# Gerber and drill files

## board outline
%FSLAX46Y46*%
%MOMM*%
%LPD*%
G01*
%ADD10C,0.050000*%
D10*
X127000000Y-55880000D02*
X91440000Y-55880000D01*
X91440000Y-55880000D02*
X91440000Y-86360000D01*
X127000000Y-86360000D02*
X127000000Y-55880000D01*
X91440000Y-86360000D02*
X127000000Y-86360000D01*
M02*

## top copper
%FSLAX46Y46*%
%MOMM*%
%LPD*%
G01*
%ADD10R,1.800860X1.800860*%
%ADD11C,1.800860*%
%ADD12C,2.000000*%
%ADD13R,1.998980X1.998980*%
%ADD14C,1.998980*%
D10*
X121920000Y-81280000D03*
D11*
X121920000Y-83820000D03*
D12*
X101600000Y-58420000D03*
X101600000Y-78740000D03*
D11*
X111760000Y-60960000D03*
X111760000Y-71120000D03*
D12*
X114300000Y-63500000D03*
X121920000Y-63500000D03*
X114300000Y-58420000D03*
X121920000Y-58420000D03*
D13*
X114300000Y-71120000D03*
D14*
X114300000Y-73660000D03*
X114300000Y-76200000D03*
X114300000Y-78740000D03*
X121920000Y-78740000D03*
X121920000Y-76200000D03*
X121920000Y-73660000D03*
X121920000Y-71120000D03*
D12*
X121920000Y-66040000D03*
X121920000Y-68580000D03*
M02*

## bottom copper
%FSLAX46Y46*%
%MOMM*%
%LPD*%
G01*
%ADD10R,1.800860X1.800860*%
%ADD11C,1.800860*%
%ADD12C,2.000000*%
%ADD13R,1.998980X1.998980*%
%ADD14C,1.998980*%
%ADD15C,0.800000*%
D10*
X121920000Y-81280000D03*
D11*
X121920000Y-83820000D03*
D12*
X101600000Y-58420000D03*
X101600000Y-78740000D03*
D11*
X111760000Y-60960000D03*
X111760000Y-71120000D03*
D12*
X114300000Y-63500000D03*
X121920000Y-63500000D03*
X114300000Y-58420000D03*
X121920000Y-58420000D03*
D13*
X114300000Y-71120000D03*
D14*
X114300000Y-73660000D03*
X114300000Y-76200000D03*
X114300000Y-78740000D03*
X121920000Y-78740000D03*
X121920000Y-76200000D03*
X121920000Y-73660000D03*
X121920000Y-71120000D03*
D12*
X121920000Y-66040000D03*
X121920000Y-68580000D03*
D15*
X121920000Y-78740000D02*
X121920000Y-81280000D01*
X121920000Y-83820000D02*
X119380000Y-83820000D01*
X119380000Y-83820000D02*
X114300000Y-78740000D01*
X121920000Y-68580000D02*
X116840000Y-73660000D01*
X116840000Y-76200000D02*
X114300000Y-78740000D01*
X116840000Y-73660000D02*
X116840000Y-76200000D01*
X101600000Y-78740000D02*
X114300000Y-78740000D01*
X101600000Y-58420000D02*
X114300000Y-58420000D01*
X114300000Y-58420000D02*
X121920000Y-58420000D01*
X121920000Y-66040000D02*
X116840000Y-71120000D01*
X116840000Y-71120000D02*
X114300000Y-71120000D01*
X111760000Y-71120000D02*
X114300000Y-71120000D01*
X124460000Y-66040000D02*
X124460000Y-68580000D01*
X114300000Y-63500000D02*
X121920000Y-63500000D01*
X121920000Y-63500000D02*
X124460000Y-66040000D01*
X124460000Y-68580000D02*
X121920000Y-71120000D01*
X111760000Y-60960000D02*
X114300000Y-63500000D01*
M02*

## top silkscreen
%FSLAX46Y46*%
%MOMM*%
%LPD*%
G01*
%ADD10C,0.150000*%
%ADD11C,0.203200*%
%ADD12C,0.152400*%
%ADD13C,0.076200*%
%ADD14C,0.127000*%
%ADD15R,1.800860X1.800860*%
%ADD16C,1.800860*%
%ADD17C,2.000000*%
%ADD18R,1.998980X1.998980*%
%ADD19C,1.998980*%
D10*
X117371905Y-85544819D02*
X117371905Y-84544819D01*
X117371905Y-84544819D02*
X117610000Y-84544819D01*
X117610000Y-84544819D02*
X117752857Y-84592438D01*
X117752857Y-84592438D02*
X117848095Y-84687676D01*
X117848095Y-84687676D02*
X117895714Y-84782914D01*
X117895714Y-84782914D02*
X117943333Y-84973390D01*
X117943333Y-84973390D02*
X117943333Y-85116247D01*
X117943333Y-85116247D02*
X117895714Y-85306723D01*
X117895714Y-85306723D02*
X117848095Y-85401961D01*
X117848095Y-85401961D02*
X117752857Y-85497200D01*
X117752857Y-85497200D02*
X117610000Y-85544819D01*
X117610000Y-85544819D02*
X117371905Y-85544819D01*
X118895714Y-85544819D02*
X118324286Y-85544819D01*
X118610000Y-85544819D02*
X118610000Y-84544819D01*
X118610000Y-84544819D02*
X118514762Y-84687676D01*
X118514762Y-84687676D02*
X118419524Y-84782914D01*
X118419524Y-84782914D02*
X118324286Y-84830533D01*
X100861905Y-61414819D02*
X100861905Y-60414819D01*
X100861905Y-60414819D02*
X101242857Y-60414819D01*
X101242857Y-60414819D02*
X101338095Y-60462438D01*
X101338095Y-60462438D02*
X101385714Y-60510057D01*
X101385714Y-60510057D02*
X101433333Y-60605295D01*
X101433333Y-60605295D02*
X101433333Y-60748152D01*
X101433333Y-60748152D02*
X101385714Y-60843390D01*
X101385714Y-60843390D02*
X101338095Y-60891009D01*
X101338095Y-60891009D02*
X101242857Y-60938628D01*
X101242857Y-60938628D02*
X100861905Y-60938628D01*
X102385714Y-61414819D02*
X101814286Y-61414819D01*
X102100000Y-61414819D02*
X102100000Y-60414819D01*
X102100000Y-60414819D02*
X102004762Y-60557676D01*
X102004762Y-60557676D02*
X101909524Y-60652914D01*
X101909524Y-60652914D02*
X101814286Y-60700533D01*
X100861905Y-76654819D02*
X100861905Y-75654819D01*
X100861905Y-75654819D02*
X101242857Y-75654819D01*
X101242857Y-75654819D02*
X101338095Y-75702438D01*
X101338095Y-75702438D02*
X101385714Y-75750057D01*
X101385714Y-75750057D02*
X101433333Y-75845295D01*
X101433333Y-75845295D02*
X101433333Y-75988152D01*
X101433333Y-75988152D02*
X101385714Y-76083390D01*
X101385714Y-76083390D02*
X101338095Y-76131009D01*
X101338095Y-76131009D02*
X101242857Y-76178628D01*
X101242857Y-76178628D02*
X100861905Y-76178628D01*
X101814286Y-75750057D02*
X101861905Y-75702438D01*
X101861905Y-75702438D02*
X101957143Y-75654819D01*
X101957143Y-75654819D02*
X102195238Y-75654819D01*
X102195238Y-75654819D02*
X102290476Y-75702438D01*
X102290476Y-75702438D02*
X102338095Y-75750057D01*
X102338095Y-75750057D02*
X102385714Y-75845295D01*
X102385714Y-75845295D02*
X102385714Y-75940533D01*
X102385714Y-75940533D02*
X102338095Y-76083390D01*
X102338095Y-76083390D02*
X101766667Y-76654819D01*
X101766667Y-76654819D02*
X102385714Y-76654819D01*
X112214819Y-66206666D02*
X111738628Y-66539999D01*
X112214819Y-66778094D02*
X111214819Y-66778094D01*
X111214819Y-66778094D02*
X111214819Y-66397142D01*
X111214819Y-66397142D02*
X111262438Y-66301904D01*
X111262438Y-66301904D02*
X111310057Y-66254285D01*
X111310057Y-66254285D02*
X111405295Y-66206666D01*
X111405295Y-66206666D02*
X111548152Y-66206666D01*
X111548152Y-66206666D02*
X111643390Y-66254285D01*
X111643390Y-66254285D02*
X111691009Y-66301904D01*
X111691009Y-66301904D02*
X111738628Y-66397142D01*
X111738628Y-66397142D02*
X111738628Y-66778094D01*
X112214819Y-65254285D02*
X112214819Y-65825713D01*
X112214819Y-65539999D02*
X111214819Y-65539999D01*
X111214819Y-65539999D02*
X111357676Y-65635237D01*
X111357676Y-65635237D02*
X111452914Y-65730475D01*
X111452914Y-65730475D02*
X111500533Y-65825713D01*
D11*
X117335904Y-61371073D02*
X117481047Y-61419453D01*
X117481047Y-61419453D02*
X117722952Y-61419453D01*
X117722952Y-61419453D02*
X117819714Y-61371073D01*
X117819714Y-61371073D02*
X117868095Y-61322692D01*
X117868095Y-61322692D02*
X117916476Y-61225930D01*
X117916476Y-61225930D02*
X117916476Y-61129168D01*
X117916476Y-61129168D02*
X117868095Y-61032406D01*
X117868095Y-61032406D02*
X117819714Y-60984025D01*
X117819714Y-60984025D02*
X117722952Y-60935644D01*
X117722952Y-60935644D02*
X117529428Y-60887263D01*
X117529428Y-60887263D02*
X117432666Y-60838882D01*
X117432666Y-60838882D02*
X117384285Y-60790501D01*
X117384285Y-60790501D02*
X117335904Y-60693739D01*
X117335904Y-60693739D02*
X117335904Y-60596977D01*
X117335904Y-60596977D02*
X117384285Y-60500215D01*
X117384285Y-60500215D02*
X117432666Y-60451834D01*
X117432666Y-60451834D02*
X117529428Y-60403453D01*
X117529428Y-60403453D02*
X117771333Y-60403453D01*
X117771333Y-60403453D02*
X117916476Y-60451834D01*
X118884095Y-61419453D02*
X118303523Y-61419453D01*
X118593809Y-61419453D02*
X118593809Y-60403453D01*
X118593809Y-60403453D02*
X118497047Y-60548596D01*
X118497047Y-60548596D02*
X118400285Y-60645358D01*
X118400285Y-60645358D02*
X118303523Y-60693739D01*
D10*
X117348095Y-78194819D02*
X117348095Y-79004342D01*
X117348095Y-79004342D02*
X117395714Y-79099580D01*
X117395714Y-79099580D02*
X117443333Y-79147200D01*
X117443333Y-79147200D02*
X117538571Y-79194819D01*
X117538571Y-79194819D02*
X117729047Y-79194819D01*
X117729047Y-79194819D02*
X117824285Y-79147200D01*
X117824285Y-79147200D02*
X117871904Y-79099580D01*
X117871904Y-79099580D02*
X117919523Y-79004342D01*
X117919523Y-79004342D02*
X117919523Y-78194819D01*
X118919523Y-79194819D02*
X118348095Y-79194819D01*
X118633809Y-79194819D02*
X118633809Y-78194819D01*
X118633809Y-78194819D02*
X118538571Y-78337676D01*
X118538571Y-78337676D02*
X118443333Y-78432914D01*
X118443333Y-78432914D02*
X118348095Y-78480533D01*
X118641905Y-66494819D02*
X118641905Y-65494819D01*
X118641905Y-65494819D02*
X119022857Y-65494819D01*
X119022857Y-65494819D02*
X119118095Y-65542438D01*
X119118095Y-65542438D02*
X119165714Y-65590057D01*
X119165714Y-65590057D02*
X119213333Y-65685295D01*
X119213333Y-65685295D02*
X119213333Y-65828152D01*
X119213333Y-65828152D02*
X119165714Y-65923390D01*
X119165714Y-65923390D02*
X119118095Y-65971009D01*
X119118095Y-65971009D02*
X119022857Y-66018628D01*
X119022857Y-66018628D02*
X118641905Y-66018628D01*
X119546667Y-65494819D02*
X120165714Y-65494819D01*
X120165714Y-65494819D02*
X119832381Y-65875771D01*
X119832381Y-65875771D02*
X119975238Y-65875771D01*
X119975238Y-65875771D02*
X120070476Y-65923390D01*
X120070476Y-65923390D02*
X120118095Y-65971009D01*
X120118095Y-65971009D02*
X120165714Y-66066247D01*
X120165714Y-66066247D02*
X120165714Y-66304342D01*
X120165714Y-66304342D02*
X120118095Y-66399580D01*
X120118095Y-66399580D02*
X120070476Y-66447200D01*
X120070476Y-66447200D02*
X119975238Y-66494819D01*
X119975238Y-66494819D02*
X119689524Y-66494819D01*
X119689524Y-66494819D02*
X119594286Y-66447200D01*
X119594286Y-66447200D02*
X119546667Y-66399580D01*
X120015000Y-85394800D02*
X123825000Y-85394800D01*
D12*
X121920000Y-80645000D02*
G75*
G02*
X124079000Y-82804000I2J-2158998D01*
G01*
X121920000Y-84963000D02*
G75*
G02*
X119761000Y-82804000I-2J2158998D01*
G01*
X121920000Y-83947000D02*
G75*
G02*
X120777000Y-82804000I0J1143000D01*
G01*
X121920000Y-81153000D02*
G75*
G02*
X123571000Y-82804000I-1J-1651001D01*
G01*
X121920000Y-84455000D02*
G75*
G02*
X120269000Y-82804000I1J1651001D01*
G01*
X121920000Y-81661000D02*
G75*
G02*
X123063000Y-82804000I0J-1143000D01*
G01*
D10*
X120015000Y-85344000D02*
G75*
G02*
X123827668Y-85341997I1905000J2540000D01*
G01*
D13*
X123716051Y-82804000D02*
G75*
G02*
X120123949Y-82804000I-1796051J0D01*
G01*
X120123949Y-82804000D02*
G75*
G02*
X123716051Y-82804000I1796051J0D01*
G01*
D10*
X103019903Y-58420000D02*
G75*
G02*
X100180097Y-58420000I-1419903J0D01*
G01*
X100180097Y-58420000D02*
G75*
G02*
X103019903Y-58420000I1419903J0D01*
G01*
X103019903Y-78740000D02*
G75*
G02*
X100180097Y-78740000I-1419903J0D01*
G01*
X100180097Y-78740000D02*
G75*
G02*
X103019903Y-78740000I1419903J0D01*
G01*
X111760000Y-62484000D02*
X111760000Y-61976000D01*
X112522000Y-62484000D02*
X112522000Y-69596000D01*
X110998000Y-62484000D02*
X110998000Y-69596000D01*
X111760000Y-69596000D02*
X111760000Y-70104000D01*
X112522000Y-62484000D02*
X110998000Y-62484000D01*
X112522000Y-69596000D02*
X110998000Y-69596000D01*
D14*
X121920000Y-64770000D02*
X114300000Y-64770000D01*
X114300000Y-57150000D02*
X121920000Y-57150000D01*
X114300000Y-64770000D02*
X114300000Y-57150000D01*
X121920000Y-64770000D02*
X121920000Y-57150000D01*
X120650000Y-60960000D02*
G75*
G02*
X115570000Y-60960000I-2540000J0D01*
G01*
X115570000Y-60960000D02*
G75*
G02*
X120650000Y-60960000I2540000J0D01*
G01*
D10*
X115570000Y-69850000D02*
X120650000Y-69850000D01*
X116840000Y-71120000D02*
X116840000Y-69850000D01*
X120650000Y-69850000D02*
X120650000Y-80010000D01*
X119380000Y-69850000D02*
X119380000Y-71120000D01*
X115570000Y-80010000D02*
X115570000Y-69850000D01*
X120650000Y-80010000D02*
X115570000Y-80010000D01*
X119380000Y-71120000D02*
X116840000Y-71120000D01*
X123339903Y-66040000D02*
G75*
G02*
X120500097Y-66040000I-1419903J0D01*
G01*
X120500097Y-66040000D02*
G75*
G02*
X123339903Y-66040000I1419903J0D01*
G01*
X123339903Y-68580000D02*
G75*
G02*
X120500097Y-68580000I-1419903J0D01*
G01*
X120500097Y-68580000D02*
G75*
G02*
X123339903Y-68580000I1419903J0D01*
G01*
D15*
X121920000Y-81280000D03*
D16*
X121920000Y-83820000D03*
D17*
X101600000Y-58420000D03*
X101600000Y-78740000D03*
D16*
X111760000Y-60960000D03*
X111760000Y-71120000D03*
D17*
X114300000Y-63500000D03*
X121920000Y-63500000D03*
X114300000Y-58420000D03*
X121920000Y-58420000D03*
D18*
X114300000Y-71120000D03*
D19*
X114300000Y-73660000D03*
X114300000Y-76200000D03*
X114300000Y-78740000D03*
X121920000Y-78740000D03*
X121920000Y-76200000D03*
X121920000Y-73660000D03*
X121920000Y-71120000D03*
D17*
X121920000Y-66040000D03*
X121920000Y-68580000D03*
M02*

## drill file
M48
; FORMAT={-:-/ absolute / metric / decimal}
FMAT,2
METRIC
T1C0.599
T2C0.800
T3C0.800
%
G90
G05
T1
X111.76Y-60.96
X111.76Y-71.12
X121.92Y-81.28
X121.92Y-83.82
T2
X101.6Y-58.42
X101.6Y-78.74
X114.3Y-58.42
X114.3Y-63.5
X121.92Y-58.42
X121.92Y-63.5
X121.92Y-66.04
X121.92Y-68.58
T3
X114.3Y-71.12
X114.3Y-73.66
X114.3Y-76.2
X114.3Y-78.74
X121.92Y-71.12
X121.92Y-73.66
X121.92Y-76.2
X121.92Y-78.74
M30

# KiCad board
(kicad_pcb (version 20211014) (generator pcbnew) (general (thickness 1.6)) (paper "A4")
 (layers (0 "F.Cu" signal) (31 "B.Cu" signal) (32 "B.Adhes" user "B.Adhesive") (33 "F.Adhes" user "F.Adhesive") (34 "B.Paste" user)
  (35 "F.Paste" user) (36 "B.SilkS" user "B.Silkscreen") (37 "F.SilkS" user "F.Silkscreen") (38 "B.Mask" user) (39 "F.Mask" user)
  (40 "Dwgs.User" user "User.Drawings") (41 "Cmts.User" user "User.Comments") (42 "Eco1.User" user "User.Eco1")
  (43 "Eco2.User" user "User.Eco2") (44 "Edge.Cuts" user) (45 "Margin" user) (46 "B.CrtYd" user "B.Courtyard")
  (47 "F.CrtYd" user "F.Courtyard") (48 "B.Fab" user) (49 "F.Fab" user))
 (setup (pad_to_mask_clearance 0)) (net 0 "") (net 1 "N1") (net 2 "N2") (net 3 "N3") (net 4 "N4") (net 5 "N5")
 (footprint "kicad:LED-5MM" (layer "F.Cu") (at 121.92 82.55 -90)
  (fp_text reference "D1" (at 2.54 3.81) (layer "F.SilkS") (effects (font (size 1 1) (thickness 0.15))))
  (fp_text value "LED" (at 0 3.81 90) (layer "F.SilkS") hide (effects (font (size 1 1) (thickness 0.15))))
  (fp_line (start 2.8448 1.905) (end 2.8448 -1.905) (layer "F.SilkS") (width 0.15))
  (fp_arc (start -1.905 0) (mid -1.272644 -1.526644) (end 0.254 -2.159) (layer "F.SilkS") (width 0.1524))
  (fp_arc (start 2.413 0) (mid 1.780644 1.526644) (end 0.254 2.159) (layer "F.SilkS") (width 0.1524))
  (fp_arc (start 1.397 0) (mid 1.062223 0.808223) (end 0.254 1.143) (layer "F.SilkS") (width 0.1524))
  (fp_arc (start -1.397 0) (mid -0.913433 -1.167433) (end 0.254 -1.651) (layer "F.SilkS") (width 0.1524))
  (fp_arc (start 1.905 0) (mid 1.421433 1.167433) (end 0.254 1.651) (layer "F.SilkS") (width 0.1524))
  (fp_arc (start -0.889 0) (mid -0.554223 -0.808223) (end 0.254 -1.143) (layer "F.SilkS") (width 0.1524))
  (fp_arc (start 2.794 1.905) (mid -2.921 0.001668) (end 2.791997 -1.907668) (layer "F.SilkS") (width 0.15))
  (fp_circle (center 0.254 0) (end -1.016 1.27) (layer "F.SilkS") (width 0.0762) (fill none))
  (pad "1" thru_hole rect locked (at -1.27 0 270) (size 1.80086 1.80086) (drill 0.59944) (layers *.Cu "F.Paste" "F.SilkS" "F.Mask")
   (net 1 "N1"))
  (pad "2" thru_hole circle locked (at 1.27 0 270) (size 1.80086 1.80086) (drill 0.59944) (layers *.Cu "F.Paste" "F.SilkS" "F.Mask")
   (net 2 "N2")))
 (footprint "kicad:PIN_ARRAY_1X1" (layer "F.Cu") (at 101.6 58.42)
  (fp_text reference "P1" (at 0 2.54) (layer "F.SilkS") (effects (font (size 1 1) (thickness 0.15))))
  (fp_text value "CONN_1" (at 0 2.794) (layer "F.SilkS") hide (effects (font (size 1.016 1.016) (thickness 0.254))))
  (fp_circle (center 0 0) (end 1.27 0.635) (layer "F.SilkS") (width 0.15) (fill none))
  (pad "1" thru_hole circle locked (at 0 0) (size 2 2) (drill 0.8) (layers *.Cu *.Mask "F.SilkS") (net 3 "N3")))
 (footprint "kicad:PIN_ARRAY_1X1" (layer "F.Cu") (at 101.6 78.74)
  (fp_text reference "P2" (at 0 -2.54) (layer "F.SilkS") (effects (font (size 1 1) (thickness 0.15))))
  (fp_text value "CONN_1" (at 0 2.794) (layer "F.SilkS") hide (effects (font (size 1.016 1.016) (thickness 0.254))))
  (fp_circle (center 0 0) (end 1.27 0.635) (layer "F.SilkS") (width 0.15) (fill none))
  (pad "1" thru_hole circle locked (at 0 0) (size 2 2) (drill 0.8) (layers *.Cu *.Mask "F.SilkS") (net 2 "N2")))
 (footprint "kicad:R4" (layer "F.Cu") (at 111.76 66.04 -90) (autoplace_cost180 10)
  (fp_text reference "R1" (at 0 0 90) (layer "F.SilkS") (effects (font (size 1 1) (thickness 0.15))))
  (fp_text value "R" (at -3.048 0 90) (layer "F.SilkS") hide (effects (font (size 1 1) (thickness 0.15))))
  (fp_line (start -3.556 0) (end -4.064 0) (layer "F.SilkS") (width 0.15))
  (fp_line (start -3.556 -0.762) (end 3.556 -0.762) (layer "F.SilkS") (width 0.15))
  (fp_line (start -3.556 0.762) (end 3.556 0.762) (layer "F.SilkS") (width 0.15))
  (fp_line (start 3.556 0) (end 4.064 0) (layer "F.SilkS") (width 0.15))
  (fp_line (start -3.556 -0.762) (end -3.556 0.762) (layer "F.SilkS") (width 0.15))
  (fp_line (start 3.556 -0.762) (end 3.556 0.762) (layer "F.SilkS") (width 0.15))
  (pad "1" thru_hole circle locked (at -5.08 0 270) (size 1.80086 1.80086) (drill 0.59944) (layers *.Cu *.Mask "F.SilkS") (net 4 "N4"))
  (pad "2" thru_hole circle locked (at 5.08 0 270) (size 1.80086 1.80086) (drill 0.59944) (layers *.Cu *.Mask "F.SilkS") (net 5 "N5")))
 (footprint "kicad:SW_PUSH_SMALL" (layer "F.Cu") (at 118.11 60.96 180)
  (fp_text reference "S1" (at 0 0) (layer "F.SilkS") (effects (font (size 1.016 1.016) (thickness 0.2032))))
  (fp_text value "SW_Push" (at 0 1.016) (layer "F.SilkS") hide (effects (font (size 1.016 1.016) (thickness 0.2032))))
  (fp_line (start -3.81 -3.81) (end 3.81 -3.81) (layer "F.SilkS") (width 0.127))
  (fp_line (start 3.81 3.81) (end -3.81 3.81) (layer "F.SilkS") (width 0.127))
  (fp_line (start 3.81 -3.81) (end 3.81 3.81) (layer "F.SilkS") (width 0.127))
  (fp_line (start -3.81 -3.81) (end -3.81 3.81) (layer "F.SilkS") (width 0.127))
  (fp_circle (center 0 0) (end 0 -2.54) (layer "F.SilkS") (width 0.127) (fill none))
  (pad "1" thru_hole circle locked (at 3.81 -2.54 180) (size 2 2) (drill 0.8) (layers *.Cu *.Mask "F.SilkS") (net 4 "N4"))
  (pad "1" thru_hole circle locked (at -3.81 -2.54 180) (size 2 2) (drill 0.8) (layers *.Cu *.Mask "F.SilkS") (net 4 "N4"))
  (pad "2" thru_hole circle locked (at 3.81 2.54 180) (size 2 2) (drill 0.8) (layers *.Cu *.Mask "F.SilkS") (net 3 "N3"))
  (pad "2" thru_hole circle locked (at -3.81 2.54 180) (size 2 2) (drill 0.8) (layers *.Cu *.Mask "F.SilkS") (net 3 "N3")))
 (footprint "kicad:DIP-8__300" (layer "F.Cu") (at 118.11 74.93 -90)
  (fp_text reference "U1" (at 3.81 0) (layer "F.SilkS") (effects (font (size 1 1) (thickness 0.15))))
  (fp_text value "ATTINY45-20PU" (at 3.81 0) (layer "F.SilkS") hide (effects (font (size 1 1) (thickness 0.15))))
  (fp_line (start -5.08 2.54) (end -5.08 -2.54) (layer "F.SilkS") (width 0.15))
  (fp_line (start -3.81 1.27) (end -5.08 1.27) (layer "F.SilkS") (width 0.15))
  (fp_line (start -5.08 -2.54) (end 5.08 -2.54) (layer "F.SilkS") (width 0.15))
  (fp_line (start -5.08 -1.27) (end -3.81 -1.27) (layer "F.SilkS") (width 0.15))
  (fp_line (start 5.08 2.54) (end -5.08 2.54) (layer "F.SilkS") (width 0.15))
  (fp_line (start 5.08 -2.54) (end 5.08 2.54) (layer "F.SilkS") (width 0.15))
  (fp_line (start -3.81 -1.27) (end -3.81 1.27) (layer "F.SilkS") (width 0.15))
  (pad "1" thru_hole rect locked (at -3.81 3.81 270) (size 1.99898 1.99898) (drill 0.8001) (layers *.Cu *.Mask "F.SilkS") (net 5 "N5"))
  (pad "2" thru_hole circle locked (at -1.27 3.81 270) (size 1.99898 1.99898) (drill 0.8001) (layers *.Cu *.Mask "F.SilkS"))
  (pad "3" thru_hole circle locked (at 1.27 3.81 270) (size 1.99898 1.99898) (drill 0.8001) (layers *.Cu *.Mask "F.SilkS"))
  (pad "4" thru_hole circle locked (at 3.81 3.81 270) (size 1.99898 1.99898) (drill 0.8001) (layers *.Cu *.Mask "F.SilkS") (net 2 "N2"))
  (pad "5" thru_hole circle locked (at 3.81 -3.81 270) (size 1.99898 1.99898) (drill 0.8001) (layers *.Cu *.Mask "F.SilkS") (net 1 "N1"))
  (pad "6" thru_hole circle locked (at 1.27 -3.81 270) (size 1.99898 1.99898) (drill 0.8001) (layers *.Cu *.Mask "F.SilkS"))
  (pad "7" thru_hole circle locked (at -1.27 -3.81 270) (size 1.99898 1.99898) (drill 0.8001) (layers *.Cu *.Mask "F.SilkS"))
  (pad "8" thru_hole circle locked (at -3.81 -3.81 270) (size 1.99898 1.99898) (drill 0.8001) (layers *.Cu *.Mask "F.SilkS") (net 4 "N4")))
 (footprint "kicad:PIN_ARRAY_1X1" (layer "F.Cu") (at 121.92 66.04)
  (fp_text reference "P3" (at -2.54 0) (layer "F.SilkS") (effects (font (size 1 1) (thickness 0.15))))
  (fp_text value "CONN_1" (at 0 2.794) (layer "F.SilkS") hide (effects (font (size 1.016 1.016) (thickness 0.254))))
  (fp_circle (center 0 0) (end 1.27 0.635) (layer "F.SilkS") (width 0.15) (fill none))
  (pad "1" thru_hole circle locked (at 0 0) (size 2 2) (drill 0.8) (layers *.Cu *.Mask "F.SilkS") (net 5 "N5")))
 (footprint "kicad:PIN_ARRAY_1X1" (layer "F.Cu") (at 121.92 68.58)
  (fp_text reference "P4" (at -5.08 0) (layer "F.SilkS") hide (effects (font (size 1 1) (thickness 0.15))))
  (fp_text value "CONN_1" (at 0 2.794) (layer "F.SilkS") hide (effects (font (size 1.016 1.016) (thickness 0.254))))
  (fp_circle (center 0 0) (end 1.27 0.635) (layer "F.SilkS") (width 0.15) (fill none))
  (pad "1" thru_hole circle locked (at 0 0) (size 2 2) (drill 0.8) (layers *.Cu *.Mask "F.SilkS") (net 2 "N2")))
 (gr_line (start 127 55.88) (end 91.44 55.88) (layer "Edge.Cuts") (width 0.05))
 (gr_line (start 91.44 55.88) (end 91.44 86.36) (layer "Edge.Cuts") (width 0.05))
 (gr_line (start 127 86.36) (end 127 55.88) (layer "Edge.Cuts") (width 0.05))
 (gr_line (start 91.44 86.36) (end 127 86.36) (layer "Edge.Cuts") (width 0.05))
 (segment (start 121.92 78.74) (end 121.92 81.28) (width 0.8) (layer "B.Cu") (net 1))
 (segment (start 121.92 83.82) (end 119.38 83.82) (width 0.8) (layer "B.Cu") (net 2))
 (segment (start 119.38 83.82) (end 114.3 78.74) (width 0.8) (layer "B.Cu") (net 2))
 (segment (start 121.92 68.58) (end 116.84 73.66) (width 0.8) (layer "B.Cu") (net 2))
 (segment (start 116.84 76.2) (end 114.3 78.74) (width 0.8) (layer "B.Cu") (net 2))
 (segment (start 116.84 73.66) (end 116.84 76.2) (width 0.8) (layer "B.Cu") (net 2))
 (segment (start 101.6 78.74) (end 114.3 78.74) (width 0.8) (layer "B.Cu") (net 2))
 (segment (start 101.6 58.42) (end 114.3 58.42) (width 0.8) (layer "B.Cu") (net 3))
 (segment (start 114.3 58.42) (end 121.92 58.42) (width 0.8) (layer "B.Cu") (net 3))
 (segment (start 121.92 66.04) (end 116.84 71.12) (width 0.8) (layer "B.Cu") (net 5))
 (segment (start 116.84 71.12) (end 114.3 71.12) (width 0.8) (layer "B.Cu") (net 5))
 (segment (start 111.76 71.12) (end 114.3 71.12) (width 0.8) (layer "B.Cu") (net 5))
 (segment (start 124.46 66.04) (end 124.46 68.58) (width 0.8) (layer "B.Cu") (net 4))
 (segment (start 114.3 63.5) (end 121.92 63.5) (width 0.8) (layer "B.Cu") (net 4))
 (segment (start 121.92 63.5) (end 124.46 66.04) (width 0.8) (layer "B.Cu") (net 4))
 (segment (start 124.46 68.58) (end 121.92 71.12) (width 0.8) (layer "B.Cu") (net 4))
 (segment (start 111.76 60.96) (end 114.3 63.5) (width 0.8) (layer "B.Cu") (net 4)))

